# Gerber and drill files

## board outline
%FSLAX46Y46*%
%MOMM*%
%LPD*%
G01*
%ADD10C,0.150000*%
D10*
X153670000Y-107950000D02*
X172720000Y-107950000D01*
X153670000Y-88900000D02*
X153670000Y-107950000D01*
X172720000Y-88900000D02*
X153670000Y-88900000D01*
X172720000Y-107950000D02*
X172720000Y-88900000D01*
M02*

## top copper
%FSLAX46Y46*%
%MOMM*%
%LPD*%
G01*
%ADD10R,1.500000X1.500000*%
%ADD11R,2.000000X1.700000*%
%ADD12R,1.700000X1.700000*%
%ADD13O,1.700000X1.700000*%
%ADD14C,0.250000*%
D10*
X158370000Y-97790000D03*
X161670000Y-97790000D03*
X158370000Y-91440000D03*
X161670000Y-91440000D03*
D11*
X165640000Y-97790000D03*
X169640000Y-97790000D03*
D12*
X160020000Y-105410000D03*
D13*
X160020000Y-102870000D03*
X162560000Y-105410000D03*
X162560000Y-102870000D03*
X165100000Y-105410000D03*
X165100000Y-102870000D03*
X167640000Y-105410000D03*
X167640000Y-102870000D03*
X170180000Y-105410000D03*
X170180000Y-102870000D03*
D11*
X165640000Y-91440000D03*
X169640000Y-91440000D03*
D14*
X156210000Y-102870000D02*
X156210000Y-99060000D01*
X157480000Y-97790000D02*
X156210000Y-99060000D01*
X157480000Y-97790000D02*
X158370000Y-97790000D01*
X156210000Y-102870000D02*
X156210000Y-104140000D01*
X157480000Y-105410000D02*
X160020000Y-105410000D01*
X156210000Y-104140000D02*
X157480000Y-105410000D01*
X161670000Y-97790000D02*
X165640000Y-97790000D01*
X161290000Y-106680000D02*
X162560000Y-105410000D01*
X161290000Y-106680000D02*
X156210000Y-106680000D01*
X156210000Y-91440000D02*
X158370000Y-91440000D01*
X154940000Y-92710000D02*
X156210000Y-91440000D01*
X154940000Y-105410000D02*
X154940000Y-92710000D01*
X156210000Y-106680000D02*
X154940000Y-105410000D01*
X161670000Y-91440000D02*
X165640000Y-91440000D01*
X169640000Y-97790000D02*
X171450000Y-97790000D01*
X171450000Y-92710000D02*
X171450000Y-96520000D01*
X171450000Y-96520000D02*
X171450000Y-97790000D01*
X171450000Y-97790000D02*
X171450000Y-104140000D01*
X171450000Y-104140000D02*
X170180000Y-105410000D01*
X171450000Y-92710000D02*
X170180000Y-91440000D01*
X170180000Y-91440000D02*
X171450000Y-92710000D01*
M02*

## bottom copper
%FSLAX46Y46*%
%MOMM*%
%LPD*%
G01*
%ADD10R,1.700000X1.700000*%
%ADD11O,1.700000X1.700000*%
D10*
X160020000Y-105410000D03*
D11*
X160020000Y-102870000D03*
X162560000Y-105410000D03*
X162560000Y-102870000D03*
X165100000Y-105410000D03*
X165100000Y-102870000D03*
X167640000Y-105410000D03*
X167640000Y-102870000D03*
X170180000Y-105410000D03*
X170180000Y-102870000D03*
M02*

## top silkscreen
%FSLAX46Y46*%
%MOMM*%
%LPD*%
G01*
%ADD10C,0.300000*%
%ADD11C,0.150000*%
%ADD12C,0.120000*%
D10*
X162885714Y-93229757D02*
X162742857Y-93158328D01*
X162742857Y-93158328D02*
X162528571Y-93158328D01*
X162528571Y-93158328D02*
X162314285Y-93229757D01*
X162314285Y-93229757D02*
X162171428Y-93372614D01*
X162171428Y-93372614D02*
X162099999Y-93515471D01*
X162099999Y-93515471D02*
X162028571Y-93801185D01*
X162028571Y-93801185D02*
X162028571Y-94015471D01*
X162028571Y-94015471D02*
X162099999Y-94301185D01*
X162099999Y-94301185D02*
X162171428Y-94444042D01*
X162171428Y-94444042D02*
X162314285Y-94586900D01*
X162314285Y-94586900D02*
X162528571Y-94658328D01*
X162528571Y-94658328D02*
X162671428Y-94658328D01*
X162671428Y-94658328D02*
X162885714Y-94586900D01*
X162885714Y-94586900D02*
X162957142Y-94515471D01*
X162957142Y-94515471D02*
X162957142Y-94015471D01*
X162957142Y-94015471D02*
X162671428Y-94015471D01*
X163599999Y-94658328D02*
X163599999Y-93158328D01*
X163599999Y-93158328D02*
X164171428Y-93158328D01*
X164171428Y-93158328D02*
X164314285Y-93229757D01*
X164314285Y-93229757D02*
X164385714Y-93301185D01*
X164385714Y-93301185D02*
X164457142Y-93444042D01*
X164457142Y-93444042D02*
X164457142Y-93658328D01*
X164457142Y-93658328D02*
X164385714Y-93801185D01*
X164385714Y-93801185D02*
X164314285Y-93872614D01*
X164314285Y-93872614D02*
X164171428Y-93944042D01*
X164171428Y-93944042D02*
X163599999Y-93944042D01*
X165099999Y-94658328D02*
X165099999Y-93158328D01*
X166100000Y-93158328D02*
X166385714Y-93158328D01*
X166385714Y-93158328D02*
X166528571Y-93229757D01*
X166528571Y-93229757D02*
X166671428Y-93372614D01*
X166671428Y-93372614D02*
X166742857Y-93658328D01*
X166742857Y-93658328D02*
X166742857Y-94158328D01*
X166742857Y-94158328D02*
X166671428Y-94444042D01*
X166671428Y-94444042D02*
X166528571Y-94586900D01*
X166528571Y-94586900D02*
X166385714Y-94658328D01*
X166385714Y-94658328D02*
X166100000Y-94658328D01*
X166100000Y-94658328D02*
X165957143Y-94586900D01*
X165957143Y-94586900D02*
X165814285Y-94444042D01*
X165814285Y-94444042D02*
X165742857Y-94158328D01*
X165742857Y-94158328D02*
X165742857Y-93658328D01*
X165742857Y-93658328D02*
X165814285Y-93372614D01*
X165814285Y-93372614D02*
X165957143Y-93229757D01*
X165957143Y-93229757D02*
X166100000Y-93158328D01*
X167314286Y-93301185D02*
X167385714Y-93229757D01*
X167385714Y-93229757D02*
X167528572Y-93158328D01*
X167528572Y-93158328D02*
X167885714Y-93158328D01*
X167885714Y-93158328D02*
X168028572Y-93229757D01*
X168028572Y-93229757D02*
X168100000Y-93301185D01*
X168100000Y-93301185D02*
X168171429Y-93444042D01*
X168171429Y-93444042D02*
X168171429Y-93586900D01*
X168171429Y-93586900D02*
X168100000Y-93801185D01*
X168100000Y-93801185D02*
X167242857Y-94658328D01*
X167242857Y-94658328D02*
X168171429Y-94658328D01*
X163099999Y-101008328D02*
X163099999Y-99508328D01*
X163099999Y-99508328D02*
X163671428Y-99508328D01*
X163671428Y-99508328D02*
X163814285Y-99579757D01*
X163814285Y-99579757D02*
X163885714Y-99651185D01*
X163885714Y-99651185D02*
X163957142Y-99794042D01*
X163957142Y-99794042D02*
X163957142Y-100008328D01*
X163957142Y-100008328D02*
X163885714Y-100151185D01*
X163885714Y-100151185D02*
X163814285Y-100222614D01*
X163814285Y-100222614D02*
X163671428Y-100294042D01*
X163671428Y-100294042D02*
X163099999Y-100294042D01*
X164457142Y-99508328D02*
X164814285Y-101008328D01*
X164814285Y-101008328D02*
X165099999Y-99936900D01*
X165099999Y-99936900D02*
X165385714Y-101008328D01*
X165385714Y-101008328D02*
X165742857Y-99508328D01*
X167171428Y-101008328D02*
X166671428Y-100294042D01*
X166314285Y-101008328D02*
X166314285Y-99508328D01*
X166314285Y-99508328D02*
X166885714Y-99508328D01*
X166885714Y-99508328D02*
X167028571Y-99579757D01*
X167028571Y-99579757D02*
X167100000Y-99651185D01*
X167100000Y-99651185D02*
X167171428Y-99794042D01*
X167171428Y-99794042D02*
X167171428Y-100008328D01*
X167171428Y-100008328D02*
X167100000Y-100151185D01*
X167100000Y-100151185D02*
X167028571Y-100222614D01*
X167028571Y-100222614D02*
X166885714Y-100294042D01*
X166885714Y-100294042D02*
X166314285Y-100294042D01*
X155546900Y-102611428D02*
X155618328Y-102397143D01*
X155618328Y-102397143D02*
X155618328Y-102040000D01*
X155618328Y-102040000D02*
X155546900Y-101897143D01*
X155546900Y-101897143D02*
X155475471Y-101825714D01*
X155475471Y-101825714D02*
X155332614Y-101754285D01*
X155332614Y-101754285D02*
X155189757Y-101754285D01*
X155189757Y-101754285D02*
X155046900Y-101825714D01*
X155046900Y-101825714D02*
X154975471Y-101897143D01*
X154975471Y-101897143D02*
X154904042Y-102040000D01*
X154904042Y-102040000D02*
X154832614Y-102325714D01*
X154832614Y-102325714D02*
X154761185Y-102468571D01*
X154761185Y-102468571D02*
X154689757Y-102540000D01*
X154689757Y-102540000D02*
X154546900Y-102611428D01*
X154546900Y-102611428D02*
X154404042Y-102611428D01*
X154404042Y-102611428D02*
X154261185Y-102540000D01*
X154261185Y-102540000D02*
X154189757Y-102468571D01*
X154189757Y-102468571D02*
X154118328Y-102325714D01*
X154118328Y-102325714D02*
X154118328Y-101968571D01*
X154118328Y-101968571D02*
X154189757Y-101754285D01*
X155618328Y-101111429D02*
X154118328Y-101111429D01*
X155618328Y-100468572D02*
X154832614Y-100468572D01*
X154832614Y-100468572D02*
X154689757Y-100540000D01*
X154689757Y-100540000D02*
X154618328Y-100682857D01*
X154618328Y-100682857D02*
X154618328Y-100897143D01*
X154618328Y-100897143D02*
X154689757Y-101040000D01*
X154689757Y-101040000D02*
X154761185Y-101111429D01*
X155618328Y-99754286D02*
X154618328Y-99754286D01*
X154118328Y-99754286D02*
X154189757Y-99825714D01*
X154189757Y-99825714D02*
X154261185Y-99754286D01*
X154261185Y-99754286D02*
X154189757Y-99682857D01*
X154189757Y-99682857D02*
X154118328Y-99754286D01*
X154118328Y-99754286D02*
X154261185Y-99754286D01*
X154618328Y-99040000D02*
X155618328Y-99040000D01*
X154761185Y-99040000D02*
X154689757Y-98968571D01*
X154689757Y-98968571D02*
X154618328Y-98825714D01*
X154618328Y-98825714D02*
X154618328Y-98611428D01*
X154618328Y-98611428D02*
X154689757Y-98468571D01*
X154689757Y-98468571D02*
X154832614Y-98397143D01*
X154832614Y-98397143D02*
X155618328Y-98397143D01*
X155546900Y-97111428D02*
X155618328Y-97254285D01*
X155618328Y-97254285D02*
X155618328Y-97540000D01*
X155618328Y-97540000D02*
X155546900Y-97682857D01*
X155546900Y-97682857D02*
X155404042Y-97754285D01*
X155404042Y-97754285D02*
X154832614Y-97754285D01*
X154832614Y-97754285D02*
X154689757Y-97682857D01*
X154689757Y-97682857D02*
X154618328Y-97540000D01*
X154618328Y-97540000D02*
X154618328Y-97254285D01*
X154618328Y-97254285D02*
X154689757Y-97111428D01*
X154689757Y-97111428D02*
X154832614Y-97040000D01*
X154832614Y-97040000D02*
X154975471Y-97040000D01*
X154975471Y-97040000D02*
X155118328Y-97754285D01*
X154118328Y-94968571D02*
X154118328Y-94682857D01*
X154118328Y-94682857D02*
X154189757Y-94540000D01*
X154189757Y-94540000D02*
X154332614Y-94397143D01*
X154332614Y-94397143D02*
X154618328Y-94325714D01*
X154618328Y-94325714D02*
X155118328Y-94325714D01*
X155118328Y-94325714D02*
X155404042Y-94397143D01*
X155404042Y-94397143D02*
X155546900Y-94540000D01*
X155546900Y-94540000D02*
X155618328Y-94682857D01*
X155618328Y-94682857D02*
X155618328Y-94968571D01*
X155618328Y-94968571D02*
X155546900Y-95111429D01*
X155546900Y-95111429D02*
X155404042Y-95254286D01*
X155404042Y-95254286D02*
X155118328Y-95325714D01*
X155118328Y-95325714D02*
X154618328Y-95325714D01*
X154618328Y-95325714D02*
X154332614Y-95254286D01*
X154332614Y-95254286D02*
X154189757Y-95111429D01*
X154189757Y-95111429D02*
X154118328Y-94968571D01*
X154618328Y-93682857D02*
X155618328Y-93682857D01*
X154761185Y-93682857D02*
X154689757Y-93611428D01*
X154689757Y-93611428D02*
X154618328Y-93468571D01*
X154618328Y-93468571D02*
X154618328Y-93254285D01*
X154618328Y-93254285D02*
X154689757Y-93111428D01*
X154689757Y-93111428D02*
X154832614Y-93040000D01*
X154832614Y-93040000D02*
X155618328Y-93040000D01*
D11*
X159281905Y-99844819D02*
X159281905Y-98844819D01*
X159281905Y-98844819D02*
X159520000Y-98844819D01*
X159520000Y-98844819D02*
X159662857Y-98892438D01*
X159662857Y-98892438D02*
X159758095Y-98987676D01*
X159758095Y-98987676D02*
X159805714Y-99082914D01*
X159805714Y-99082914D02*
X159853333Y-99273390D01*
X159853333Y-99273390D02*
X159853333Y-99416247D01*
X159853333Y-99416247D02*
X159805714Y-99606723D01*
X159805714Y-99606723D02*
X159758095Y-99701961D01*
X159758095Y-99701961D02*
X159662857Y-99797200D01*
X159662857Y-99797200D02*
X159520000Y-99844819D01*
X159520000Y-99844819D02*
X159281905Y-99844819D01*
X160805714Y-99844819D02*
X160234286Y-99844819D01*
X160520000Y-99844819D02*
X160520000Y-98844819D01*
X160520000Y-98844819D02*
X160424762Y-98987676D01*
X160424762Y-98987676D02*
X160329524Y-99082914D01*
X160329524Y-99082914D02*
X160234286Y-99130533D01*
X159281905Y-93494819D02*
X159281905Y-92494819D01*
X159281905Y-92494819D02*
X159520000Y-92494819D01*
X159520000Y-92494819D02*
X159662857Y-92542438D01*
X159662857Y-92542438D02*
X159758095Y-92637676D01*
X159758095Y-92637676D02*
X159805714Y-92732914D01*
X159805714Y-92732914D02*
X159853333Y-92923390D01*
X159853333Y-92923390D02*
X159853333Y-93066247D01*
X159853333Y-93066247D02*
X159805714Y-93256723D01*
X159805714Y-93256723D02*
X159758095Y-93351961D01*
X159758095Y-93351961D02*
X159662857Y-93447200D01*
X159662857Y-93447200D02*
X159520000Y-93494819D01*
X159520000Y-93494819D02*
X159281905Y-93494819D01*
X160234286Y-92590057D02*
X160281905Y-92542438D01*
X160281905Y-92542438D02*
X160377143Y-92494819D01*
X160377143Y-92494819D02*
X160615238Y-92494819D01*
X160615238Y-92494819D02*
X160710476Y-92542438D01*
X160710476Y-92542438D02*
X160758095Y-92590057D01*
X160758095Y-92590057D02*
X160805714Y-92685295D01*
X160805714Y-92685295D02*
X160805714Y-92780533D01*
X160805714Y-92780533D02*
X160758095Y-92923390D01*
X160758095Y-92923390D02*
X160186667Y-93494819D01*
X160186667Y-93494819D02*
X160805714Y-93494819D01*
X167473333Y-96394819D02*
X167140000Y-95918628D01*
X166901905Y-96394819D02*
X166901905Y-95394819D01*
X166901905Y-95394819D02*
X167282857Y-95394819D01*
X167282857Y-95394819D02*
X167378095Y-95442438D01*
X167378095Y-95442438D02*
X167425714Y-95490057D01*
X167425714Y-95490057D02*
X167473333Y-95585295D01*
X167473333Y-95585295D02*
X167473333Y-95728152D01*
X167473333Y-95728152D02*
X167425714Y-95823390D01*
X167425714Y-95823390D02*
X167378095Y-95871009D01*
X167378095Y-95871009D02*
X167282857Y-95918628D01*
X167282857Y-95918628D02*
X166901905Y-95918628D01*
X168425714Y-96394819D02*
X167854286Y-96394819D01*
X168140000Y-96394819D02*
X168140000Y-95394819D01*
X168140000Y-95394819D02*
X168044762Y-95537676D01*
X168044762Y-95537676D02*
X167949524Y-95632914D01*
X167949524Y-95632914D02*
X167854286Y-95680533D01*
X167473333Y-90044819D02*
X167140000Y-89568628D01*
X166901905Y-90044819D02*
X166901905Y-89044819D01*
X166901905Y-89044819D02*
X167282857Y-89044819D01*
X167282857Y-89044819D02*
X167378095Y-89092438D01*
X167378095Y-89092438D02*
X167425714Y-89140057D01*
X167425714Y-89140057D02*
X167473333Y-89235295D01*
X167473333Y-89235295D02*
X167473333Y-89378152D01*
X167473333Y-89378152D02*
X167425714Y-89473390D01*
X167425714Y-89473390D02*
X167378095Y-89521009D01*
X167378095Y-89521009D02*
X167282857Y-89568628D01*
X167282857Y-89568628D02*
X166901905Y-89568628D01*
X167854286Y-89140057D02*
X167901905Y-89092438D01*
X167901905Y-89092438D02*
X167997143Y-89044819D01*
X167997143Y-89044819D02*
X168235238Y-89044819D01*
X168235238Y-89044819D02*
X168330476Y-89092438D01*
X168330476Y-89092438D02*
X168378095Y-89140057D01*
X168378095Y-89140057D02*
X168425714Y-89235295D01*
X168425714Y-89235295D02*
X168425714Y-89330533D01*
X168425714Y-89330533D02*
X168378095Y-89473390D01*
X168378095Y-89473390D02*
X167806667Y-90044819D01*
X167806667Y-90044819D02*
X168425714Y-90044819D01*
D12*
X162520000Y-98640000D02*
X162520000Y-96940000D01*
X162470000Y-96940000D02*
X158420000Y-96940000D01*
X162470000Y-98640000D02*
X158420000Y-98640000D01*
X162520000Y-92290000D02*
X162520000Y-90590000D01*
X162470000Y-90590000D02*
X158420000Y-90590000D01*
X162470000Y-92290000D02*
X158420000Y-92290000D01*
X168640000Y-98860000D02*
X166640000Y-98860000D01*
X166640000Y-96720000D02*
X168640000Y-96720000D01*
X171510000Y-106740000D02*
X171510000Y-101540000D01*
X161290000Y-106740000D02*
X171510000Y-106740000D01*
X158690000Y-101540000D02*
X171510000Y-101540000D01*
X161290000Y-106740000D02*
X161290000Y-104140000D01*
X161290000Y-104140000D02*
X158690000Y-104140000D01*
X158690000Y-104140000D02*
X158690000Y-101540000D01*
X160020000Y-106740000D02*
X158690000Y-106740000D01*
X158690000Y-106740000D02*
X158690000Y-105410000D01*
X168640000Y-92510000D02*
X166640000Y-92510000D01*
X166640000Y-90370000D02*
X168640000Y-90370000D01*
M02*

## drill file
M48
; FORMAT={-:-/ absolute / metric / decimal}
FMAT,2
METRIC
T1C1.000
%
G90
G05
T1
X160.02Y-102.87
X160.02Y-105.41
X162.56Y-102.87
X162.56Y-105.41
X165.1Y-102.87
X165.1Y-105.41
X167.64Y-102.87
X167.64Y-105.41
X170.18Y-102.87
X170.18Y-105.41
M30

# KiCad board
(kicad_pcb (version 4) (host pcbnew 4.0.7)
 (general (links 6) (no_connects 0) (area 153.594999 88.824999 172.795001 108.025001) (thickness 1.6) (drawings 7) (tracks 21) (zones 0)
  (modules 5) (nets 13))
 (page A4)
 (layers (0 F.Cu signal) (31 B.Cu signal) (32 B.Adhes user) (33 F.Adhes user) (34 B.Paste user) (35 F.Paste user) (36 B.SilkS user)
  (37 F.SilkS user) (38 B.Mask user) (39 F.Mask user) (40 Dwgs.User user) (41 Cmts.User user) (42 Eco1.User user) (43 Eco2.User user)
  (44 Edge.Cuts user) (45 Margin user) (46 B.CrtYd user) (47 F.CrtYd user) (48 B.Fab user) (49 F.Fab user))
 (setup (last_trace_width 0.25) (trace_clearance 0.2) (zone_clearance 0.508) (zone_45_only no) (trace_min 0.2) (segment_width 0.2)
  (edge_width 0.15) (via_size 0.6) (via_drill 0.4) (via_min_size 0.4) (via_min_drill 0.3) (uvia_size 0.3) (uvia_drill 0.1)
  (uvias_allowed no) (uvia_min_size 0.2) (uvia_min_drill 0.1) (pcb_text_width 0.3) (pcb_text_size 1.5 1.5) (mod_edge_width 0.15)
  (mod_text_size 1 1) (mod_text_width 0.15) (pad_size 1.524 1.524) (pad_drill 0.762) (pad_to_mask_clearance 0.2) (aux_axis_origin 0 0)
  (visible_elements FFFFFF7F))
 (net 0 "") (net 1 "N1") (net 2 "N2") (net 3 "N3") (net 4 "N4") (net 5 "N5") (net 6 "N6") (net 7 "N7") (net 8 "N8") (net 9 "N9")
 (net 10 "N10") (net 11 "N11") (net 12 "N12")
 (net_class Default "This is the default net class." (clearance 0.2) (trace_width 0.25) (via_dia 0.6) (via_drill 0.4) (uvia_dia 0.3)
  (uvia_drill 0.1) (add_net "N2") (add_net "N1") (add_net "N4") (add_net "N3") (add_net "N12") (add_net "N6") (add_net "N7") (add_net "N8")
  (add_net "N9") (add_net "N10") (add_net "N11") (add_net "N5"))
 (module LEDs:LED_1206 (layer F.Cu) (at 160.02 97.79 180)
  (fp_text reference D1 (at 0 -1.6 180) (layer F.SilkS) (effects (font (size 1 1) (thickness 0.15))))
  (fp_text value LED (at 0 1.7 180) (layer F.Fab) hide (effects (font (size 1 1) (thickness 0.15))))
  (fp_line (start -2.5 -0.85) (end -2.5 0.85) (layer F.SilkS) (width 0.12))
  (fp_line (start -2.45 0.85) (end 1.6 0.85) (layer F.SilkS) (width 0.12))
  (fp_line (start -2.45 -0.85) (end 1.6 -0.85) (layer F.SilkS) (width 0.12))
  (pad 2 smd rect (at 1.65 0) (size 1.5 1.5) (layers F.Cu F.Paste F.Mask) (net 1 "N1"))
  (pad 1 smd rect (at -1.65 0) (size 1.5 1.5) (layers F.Cu F.Paste F.Mask) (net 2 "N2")))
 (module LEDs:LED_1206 (layer F.Cu) (at 160.02 91.44 180)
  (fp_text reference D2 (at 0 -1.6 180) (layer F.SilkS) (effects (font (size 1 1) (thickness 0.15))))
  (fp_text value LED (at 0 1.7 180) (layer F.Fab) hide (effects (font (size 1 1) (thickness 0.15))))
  (fp_line (start -2.5 -0.85) (end -2.5 0.85) (layer F.SilkS) (width 0.12))
  (fp_line (start -2.45 0.85) (end 1.6 0.85) (layer F.SilkS) (width 0.12))
  (fp_line (start -2.45 -0.85) (end 1.6 -0.85) (layer F.SilkS) (width 0.12))
  (pad 2 smd rect (at 1.65 0) (size 1.5 1.5) (layers F.Cu F.Paste F.Mask) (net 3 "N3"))
  (pad 1 smd rect (at -1.65 0) (size 1.5 1.5) (layers F.Cu F.Paste F.Mask) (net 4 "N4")))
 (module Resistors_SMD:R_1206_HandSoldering (layer F.Cu) (at 167.64 97.79)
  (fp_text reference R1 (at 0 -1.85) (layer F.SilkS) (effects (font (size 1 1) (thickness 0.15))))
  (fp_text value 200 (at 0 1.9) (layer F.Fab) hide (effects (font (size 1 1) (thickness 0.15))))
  (fp_line (start 1 1.07) (end -1 1.07) (layer F.SilkS) (width 0.12))
  (fp_line (start -1 -1.07) (end 1 -1.07) (layer F.SilkS) (width 0.12))
  (pad 1 smd rect (at -2 0) (size 2 1.7) (layers F.Cu F.Paste F.Mask) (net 2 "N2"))
  (pad 2 smd rect (at 2 0) (size 2 1.7) (layers F.Cu F.Paste F.Mask) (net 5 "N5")))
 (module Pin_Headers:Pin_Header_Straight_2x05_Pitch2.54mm (layer F.Cu) (at 160.02 105.41 90)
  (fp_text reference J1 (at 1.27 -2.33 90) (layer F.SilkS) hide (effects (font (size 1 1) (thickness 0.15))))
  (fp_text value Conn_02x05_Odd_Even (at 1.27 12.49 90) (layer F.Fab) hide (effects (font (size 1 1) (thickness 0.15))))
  (fp_line (start -1.33 11.49) (end 3.87 11.49) (layer F.SilkS) (width 0.12))
  (fp_line (start -1.33 1.27) (end -1.33 11.49) (layer F.SilkS) (width 0.12))
  (fp_line (start 3.87 -1.33) (end 3.87 11.49) (layer F.SilkS) (width 0.12))
  (fp_line (start -1.33 1.27) (end 1.27 1.27) (layer F.SilkS) (width 0.12))
  (fp_line (start 1.27 1.27) (end 1.27 -1.33) (layer F.SilkS) (width 0.12))
  (fp_line (start 1.27 -1.33) (end 3.87 -1.33) (layer F.SilkS) (width 0.12))
  (fp_line (start -1.33 0) (end -1.33 -1.33) (layer F.SilkS) (width 0.12))
  (fp_line (start -1.33 -1.33) (end 0 -1.33) (layer F.SilkS) (width 0.12))
  (pad 1 thru_hole rect (at 0 0 90) (size 1.7 1.7) (drill 1) (layers *.Cu *.Mask) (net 1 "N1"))
  (pad 2 thru_hole oval (at 2.54 0 90) (size 1.7 1.7) (drill 1) (layers *.Cu *.Mask) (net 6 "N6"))
  (pad 3 thru_hole oval (at 0 2.54 90) (size 1.7 1.7) (drill 1) (layers *.Cu *.Mask) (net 3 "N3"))
  (pad 4 thru_hole oval (at 2.54 2.54 90) (size 1.7 1.7) (drill 1) (layers *.Cu *.Mask) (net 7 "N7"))
  (pad 5 thru_hole oval (at 0 5.08 90) (size 1.7 1.7) (drill 1) (layers *.Cu *.Mask) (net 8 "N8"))
  (pad 6 thru_hole oval (at 2.54 5.08 90) (size 1.7 1.7) (drill 1) (layers *.Cu *.Mask) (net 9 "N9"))
  (pad 7 thru_hole oval (at 0 7.62 90) (size 1.7 1.7) (drill 1) (layers *.Cu *.Mask) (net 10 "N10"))
  (pad 8 thru_hole oval (at 2.54 7.62 90) (size 1.7 1.7) (drill 1) (layers *.Cu *.Mask) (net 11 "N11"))
  (pad 9 thru_hole oval (at 0 10.16 90) (size 1.7 1.7) (drill 1) (layers *.Cu *.Mask) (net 5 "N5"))
  (pad 10 thru_hole oval (at 2.54 10.16 90) (size 1.7 1.7) (drill 1) (layers *.Cu *.Mask) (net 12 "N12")))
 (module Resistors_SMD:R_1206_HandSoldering (layer F.Cu) (at 167.64 91.44)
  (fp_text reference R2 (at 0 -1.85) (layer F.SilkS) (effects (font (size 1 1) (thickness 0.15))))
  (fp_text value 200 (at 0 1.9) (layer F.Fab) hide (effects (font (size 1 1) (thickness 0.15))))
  (fp_line (start 1 1.07) (end -1 1.07) (layer F.SilkS) (width 0.12))
  (fp_line (start -1 -1.07) (end 1 -1.07) (layer F.SilkS) (width 0.12))
  (pad 1 smd rect (at -2 0) (size 2 1.7) (layers F.Cu F.Paste F.Mask) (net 4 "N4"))
  (pad 2 smd rect (at 2 0) (size 2 1.7) (layers F.Cu F.Paste F.Mask) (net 5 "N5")))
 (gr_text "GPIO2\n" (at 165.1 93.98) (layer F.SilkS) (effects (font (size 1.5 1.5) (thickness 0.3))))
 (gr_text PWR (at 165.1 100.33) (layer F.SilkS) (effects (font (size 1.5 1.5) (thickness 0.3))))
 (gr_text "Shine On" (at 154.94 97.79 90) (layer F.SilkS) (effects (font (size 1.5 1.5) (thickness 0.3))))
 (gr_line (start 153.67 107.95) (end 172.72 107.95) (angle 90) (layer Edge.Cuts) (width 0.15))
 (gr_line (start 153.67 88.9) (end 153.67 107.95) (angle 90) (layer Edge.Cuts) (width 0.15))
 (gr_line (start 172.72 88.9) (end 153.67 88.9) (angle 90) (layer Edge.Cuts) (width 0.15))
 (gr_line (start 172.72 107.95) (end 172.72 88.9) (angle 90) (layer Edge.Cuts) (width 0.15))
 (segment (start 156.21 102.87) (end 156.21 99.06) (width 0.25) (layer F.Cu) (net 1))
 (segment (start 157.48 97.79) (end 156.21 99.06) (width 0.25) (layer F.Cu) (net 1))
 (segment (start 157.48 97.79) (end 158.37 97.79) (width 0.25) (layer F.Cu) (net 1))
 (segment (start 156.21 102.87) (end 156.21 104.14) (width 0.25) (layer F.Cu) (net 1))
 (segment (start 157.48 105.41) (end 160.02 105.41) (width 0.25) (layer F.Cu) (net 1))
 (segment (start 156.21 104.14) (end 157.48 105.41) (width 0.25) (layer F.Cu) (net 1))
 (segment (start 161.67 97.79) (end 165.64 97.79) (width 0.25) (layer F.Cu) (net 2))
 (segment (start 161.29 106.68) (end 162.56 105.41) (width 0.25) (layer F.Cu) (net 3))
 (segment (start 161.29 106.68) (end 156.21 106.68) (width 0.25) (layer F.Cu) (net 3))
 (segment (start 156.21 91.44) (end 158.37 91.44) (width 0.25) (layer F.Cu) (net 3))
 (segment (start 154.94 92.71) (end 156.21 91.44) (width 0.25) (layer F.Cu) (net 3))
 (segment (start 154.94 105.41) (end 154.94 92.71) (width 0.25) (layer F.Cu) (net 3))
 (segment (start 156.21 106.68) (end 154.94 105.41) (width 0.25) (layer F.Cu) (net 3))
 (segment (start 161.67 91.44) (end 165.64 91.44) (width 0.25) (layer F.Cu) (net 4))
 (segment (start 169.64 97.79) (end 171.45 97.79) (width 0.25) (layer F.Cu) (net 5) (status 400000))
 (segment (start 171.45 92.71) (end 171.45 96.52) (width 0.25) (layer F.Cu) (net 5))
 (segment (start 171.45 96.52) (end 171.45 97.79) (width 0.25) (layer F.Cu) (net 5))
 (segment (start 171.45 97.79) (end 171.45 104.14) (width 0.25) (layer F.Cu) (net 5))
 (segment (start 171.45 104.14) (end 170.18 105.41) (width 0.25) (layer F.Cu) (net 5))
 (segment (start 171.45 92.71) (end 170.18 91.44) (width 0.25) (layer F.Cu) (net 5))
 (segment (start 170.18 91.44) (end 171.45 92.71) (width 0.25) (layer F.Cu) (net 5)))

